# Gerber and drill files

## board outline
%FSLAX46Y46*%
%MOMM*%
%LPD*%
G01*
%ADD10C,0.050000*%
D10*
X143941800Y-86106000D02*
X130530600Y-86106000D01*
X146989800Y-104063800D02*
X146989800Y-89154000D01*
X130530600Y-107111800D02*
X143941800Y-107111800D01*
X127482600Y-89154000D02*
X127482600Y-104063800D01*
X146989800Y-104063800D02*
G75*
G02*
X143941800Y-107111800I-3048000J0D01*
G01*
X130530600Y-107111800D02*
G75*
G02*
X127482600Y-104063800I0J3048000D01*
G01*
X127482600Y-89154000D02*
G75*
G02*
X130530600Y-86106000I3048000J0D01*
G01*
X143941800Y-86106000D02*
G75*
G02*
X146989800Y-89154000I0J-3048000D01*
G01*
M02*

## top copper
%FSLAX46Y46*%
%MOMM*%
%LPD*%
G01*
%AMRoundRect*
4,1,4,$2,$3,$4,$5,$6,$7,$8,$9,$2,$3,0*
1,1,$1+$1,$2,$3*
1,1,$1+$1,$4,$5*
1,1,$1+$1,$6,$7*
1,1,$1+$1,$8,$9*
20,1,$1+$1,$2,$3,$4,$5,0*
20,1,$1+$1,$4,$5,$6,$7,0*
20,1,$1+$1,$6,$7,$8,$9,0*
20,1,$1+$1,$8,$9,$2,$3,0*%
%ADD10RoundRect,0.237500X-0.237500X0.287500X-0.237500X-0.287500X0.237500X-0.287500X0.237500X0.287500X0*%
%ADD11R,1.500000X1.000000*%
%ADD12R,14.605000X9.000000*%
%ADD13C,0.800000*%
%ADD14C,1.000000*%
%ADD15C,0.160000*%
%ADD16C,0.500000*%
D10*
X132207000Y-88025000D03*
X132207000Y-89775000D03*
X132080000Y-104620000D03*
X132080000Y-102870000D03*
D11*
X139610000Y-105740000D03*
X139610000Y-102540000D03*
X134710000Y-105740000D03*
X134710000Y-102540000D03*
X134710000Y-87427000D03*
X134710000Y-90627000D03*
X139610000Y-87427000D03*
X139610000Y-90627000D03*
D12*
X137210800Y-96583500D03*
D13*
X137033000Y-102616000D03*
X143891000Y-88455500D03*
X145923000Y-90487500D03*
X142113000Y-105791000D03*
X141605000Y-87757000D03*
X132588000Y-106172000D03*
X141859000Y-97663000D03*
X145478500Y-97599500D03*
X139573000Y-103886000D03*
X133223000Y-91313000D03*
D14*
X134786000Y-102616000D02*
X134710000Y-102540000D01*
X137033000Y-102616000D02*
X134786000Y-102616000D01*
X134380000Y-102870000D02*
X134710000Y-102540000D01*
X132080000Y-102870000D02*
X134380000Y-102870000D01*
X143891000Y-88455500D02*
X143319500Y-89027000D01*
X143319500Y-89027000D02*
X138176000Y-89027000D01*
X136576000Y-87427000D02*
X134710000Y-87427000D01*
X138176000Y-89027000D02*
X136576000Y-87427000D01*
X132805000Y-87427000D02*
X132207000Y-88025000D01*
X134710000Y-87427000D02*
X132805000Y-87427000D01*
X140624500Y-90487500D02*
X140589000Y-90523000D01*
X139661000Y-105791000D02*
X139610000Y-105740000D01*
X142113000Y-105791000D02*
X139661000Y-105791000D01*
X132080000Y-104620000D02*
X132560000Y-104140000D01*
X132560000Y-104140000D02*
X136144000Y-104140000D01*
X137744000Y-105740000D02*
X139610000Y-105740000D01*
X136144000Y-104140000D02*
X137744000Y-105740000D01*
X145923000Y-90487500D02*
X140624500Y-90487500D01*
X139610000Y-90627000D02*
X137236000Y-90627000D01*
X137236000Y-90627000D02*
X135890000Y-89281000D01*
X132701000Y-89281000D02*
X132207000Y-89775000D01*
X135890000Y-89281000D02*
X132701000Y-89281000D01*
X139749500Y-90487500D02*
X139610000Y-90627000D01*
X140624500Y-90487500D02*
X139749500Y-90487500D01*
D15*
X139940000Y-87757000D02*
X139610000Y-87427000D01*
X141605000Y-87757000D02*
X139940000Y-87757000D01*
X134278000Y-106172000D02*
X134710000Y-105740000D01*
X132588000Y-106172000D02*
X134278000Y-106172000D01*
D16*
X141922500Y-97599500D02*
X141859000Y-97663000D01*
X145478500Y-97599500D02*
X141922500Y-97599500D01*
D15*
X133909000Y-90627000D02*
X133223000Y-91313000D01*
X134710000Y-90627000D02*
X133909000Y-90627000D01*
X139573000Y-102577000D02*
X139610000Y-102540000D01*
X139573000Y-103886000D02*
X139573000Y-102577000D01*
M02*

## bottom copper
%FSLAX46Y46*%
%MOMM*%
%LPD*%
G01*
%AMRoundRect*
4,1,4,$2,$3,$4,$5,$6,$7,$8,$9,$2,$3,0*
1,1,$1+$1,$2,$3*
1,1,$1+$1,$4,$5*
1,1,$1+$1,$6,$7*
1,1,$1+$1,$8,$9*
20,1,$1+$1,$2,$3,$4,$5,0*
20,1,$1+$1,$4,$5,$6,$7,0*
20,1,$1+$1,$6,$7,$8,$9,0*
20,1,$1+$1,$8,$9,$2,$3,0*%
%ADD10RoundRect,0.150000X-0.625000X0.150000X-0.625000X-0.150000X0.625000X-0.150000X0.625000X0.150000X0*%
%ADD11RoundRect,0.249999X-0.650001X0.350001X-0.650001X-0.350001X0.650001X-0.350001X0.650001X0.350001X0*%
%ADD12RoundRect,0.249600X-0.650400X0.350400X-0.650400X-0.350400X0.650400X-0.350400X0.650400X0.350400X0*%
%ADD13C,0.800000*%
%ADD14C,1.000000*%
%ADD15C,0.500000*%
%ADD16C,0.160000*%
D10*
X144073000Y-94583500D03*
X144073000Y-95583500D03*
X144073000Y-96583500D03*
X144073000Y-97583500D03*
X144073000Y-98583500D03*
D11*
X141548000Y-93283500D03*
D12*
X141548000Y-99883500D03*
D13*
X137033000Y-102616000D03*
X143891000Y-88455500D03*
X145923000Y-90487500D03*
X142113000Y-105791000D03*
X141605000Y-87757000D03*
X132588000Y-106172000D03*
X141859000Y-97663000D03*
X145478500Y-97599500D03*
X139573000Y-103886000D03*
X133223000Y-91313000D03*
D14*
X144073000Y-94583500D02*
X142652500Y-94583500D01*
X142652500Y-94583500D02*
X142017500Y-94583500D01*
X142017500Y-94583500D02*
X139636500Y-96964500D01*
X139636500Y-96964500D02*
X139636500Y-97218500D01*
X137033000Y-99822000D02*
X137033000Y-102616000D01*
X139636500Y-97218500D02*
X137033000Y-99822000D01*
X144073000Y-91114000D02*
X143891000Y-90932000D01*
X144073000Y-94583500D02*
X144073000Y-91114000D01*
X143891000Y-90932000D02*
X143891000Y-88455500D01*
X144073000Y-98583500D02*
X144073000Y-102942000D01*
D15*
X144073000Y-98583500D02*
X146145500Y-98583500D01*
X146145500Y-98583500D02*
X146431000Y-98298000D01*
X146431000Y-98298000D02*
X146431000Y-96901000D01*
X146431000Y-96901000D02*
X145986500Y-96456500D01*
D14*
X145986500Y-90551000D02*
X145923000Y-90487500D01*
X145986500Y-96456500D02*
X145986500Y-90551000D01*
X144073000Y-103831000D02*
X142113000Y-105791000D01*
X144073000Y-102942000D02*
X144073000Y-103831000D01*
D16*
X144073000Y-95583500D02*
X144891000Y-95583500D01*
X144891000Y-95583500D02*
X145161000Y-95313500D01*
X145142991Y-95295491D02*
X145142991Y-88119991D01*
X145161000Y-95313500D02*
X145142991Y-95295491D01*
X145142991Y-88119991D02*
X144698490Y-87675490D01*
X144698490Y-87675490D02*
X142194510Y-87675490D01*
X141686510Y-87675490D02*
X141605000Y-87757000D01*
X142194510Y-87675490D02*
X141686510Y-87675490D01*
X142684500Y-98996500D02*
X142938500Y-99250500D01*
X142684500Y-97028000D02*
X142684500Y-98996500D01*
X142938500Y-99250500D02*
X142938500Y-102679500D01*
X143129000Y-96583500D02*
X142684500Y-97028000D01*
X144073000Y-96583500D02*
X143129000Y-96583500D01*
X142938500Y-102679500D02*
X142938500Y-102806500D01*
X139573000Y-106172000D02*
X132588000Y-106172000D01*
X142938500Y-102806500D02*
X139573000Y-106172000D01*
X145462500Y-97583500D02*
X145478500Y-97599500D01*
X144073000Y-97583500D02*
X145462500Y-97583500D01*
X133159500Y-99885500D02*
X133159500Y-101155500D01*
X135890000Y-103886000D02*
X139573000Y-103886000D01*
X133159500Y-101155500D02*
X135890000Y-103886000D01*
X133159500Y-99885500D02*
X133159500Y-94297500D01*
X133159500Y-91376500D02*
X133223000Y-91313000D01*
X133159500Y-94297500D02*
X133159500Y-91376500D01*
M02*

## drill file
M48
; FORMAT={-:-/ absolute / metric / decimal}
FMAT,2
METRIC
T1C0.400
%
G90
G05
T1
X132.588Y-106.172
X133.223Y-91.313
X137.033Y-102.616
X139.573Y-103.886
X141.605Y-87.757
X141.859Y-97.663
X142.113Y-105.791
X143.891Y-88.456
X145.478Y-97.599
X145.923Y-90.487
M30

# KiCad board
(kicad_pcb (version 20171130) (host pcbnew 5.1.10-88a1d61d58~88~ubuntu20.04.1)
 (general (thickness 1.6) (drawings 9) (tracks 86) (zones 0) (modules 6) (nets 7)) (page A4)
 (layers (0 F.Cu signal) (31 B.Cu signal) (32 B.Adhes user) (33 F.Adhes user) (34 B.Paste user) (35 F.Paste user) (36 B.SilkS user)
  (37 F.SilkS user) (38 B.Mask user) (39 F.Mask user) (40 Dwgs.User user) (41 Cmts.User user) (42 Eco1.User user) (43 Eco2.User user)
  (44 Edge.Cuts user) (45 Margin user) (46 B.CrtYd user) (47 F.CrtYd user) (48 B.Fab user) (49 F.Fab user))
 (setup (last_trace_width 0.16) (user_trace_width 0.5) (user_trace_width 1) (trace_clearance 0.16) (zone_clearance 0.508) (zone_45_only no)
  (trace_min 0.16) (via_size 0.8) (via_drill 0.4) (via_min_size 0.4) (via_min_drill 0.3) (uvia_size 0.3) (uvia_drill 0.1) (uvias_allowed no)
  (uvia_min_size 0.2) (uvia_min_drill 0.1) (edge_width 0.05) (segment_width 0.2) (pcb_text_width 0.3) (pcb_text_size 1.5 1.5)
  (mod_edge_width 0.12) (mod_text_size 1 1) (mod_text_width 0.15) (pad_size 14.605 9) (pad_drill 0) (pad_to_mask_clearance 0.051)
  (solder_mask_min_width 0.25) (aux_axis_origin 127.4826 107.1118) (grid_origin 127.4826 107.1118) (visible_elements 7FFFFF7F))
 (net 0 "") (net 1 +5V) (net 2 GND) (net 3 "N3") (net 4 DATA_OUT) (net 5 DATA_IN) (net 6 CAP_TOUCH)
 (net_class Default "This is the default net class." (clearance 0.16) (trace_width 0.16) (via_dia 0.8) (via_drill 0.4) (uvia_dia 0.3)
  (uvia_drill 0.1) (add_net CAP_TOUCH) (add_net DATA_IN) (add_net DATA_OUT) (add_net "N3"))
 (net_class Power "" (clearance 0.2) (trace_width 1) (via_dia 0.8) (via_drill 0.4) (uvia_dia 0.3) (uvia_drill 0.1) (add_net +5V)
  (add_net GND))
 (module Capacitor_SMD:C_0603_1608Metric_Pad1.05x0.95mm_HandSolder (layer F.Cu) (at 132.207 88.9 270)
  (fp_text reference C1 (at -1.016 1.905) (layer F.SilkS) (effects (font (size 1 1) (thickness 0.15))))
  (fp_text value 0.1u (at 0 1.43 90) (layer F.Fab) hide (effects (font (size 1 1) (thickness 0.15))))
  (pad 1 smd roundrect (at -0.875 0 270) (size 1.05 0.95) (layers F.Cu F.Paste F.Mask) (roundrect_rratio 0.25) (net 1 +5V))
  (pad 2 smd roundrect (at 0.875 0 270) (size 1.05 0.95) (layers F.Cu F.Mask) (roundrect_rratio 0.25) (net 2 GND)))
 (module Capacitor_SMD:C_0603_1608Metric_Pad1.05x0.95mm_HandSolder (layer F.Cu) (at 132.08 103.745 270)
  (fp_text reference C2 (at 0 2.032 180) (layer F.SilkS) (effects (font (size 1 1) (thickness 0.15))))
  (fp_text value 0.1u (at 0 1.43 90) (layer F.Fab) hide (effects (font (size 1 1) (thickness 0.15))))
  (pad 2 smd roundrect (at 0.875 0 270) (size 1.05 0.95) (layers F.Cu F.Mask) (roundrect_rratio 0.25) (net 2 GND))
  (pad 1 smd roundrect (at -0.875 0 270) (size 1.05 0.95) (layers F.Cu F.Paste F.Mask) (roundrect_rratio 0.25) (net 1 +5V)))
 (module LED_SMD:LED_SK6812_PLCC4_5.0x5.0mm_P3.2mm (layer F.Cu) (at 137.16 104.14)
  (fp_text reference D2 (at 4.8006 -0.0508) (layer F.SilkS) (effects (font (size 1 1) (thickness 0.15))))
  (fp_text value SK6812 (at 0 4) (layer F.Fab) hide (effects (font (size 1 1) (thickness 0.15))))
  (pad 1 smd rect (at 2.45 1.6) (size 1.5 1) (layers F.Cu F.Mask) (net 2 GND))
  (pad 2 smd rect (at 2.45 -1.6) (size 1.5 1) (layers F.Cu F.Mask) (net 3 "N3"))
  (pad 4 smd rect (at -2.45 1.6) (size 1.5 1) (layers F.Cu F.Mask) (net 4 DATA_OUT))
  (pad 3 smd rect (at -2.45 -1.6) (size 1.5 1) (layers F.Cu F.Paste F.Mask) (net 1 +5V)))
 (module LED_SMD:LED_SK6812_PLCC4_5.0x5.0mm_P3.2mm (layer F.Cu) (at 137.16 89.027)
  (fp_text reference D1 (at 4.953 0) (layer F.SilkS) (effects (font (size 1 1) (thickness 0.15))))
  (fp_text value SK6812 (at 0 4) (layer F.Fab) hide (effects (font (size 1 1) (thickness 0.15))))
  (pad 3 smd rect (at -2.45 -1.6) (size 1.5 1) (layers F.Cu F.Paste F.Mask) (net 1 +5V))
  (pad 4 smd rect (at -2.45 1.6) (size 1.5 1) (layers F.Cu F.Mask) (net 3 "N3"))
  (pad 2 smd rect (at 2.45 -1.6) (size 1.5 1) (layers F.Cu F.Mask) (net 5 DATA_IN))
  (pad 1 smd rect (at 2.45 1.6) (size 1.5 1) (layers F.Cu F.Mask) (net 2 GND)))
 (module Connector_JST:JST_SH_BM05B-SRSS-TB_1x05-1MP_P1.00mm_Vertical (layer B.Cu) (at 142.748 96.5835 270)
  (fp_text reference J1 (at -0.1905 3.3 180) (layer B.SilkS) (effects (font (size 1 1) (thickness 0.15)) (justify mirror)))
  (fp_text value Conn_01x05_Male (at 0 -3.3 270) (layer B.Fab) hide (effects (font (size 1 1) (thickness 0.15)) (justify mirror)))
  (pad 1 smd roundrect (at -2 -1.325 270) (size 0.6 1.55) (layers B.Cu B.Mask) (roundrect_rratio 0.25) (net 1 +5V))
  (pad 2 smd roundrect (at -1 -1.325 270) (size 0.6 1.55) (layers B.Cu B.Mask) (roundrect_rratio 0.25) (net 5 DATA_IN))
  (pad 3 smd roundrect (at 0 -1.325 270) (size 0.6 1.55) (layers B.Cu B.Mask) (roundrect_rratio 0.25) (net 4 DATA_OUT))
  (pad 4 smd roundrect (at 1 -1.325 270) (size 0.6 1.55) (layers B.Cu B.Mask) (roundrect_rratio 0.25) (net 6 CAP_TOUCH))
  (pad 5 smd roundrect (at 2 -1.325 270) (size 0.6 1.55) (layers B.Cu B.Mask) (roundrect_rratio 0.25) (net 2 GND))
  (pad MP smd roundrect (at -3.3 1.2 270) (size 1.2 1.8) (layers B.Cu B.Paste B.Mask) (roundrect_rratio 0.2083325))
  (pad MP smd roundrect (at 3.3 1.2 270) (size 1.2 1.8) (layers B.Cu B.Mask) (roundrect_rratio 0.208)))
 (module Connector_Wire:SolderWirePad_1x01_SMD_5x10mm (layer F.Cu) (at 136.0805 96.647)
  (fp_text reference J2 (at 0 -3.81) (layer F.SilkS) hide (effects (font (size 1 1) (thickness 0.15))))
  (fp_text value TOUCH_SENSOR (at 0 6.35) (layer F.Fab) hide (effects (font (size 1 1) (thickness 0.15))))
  (pad 1 smd rect (at 1.1303 -0.0635) (size 14.605 9) (layers F.Cu F.Mask) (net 6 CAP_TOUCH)))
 (gr_line (start 143.9418 86.106) (end 130.5306 86.106) (layer Edge.Cuts) (width 0.05))
 (gr_line (start 146.9898 104.0638) (end 146.9898 89.154) (layer Edge.Cuts) (width 0.05))
 (gr_line (start 130.5306 107.1118) (end 143.9418 107.1118) (layer Edge.Cuts) (width 0.05))
 (gr_line (start 127.4826 89.154) (end 127.4826 104.0638) (layer Edge.Cuts) (width 0.05))
 (gr_arc (start 143.9418 104.0638) (end 143.9418 107.1118) (angle -90) (layer Edge.Cuts) (width 0.05))
 (gr_arc (start 130.5306 104.0638) (end 127.4826 104.0638) (angle -90) (layer Edge.Cuts) (width 0.05))
 (gr_arc (start 130.5306 89.154) (end 130.5306 86.106) (angle -90) (layer Edge.Cuts) (width 0.05))
 (gr_arc (start 143.9418 89.154) (end 146.9898 89.154) (angle -90) (layer Edge.Cuts) (width 0.05))
 (segment (start 144.073 94.5835) (end 142.6525 94.5835) (width 1) (layer B.Cu) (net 1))
 (segment (start 142.6525 94.5835) (end 142.0175 94.5835) (width 1) (layer B.Cu) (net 1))
 (segment (start 142.0175 94.5835) (end 139.6365 96.9645) (width 1) (layer B.Cu) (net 1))
 (segment (start 139.6365 96.9645) (end 139.6365 97.2185) (width 1) (layer B.Cu) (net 1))
 (via (at 137.033 102.616) (size 0.8) (drill 0.4) (layers F.Cu B.Cu) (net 1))
 (segment (start 137.033 99.822) (end 137.033 102.616) (width 1) (layer B.Cu) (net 1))
 (segment (start 139.6365 97.2185) (end 137.033 99.822) (width 1) (layer B.Cu) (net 1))
 (segment (start 134.786 102.616) (end 134.71 102.54) (width 1) (layer F.Cu) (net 1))
 (segment (start 137.033 102.616) (end 134.786 102.616) (width 1) (layer F.Cu) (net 1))
 (segment (start 134.38 102.87) (end 134.71 102.54) (width 1) (layer F.Cu) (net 1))
 (segment (start 132.08 102.87) (end 134.38 102.87) (width 1) (layer F.Cu) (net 1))
 (via (at 143.891 88.4555) (size 0.8) (drill 0.4) (layers F.Cu B.Cu) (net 1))
 (segment (start 144.073 91.114) (end 143.891 90.932) (width 1) (layer B.Cu) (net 1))
 (segment (start 144.073 94.5835) (end 144.073 91.114) (width 1) (layer B.Cu) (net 1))
 (segment (start 143.891 90.932) (end 143.891 88.4555) (width 1) (layer B.Cu) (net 1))
 (segment (start 143.891 88.4555) (end 143.3195 89.027) (width 1) (layer F.Cu) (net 1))
 (segment (start 143.3195 89.027) (end 138.176 89.027) (width 1) (layer F.Cu) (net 1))
 (segment (start 136.576 87.427) (end 134.71 87.427) (width 1) (layer F.Cu) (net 1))
 (segment (start 138.176 89.027) (end 136.576 87.427) (width 1) (layer F.Cu) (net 1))
 (segment (start 132.805 87.427) (end 132.207 88.025) (width 1) (layer F.Cu) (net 1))
 (segment (start 134.71 87.427) (end 132.805 87.427) (width 1) (layer F.Cu) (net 1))
 (segment (start 144.073 98.5835) (end 144.073 102.942) (width 1) (layer B.Cu) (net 2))
 (segment (start 144.073 98.5835) (end 146.1455 98.5835) (width 0.5) (layer B.Cu) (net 2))
 (segment (start 146.1455 98.5835) (end 146.431 98.298) (width 0.5) (layer B.Cu) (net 2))
 (segment (start 146.431 98.298) (end 146.431 96.901) (width 0.5) (layer B.Cu) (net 2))
 (segment (start 146.431 96.901) (end 145.9865 96.4565) (width 0.5) (layer B.Cu) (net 2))
 (via (at 145.923 90.4875) (size 0.8) (drill 0.4) (layers F.Cu B.Cu) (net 2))
 (segment (start 140.6245 90.4875) (end 140.589 90.523) (width 1) (layer F.Cu) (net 2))
 (segment (start 145.9865 90.551) (end 145.923 90.4875) (width 1) (layer B.Cu) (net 2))
 (segment (start 145.9865 96.4565) (end 145.9865 90.551) (width 1) (layer B.Cu) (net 2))
 (via (at 142.113 105.791) (size 0.8) (drill 0.4) (layers F.Cu B.Cu) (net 2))
 (segment (start 144.073 103.831) (end 142.113 105.791) (width 1) (layer B.Cu) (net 2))
 (segment (start 144.073 102.942) (end 144.073 103.831) (width 1) (layer B.Cu) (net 2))
 (segment (start 139.661 105.791) (end 139.61 105.74) (width 1) (layer F.Cu) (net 2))
 (segment (start 142.113 105.791) (end 139.661 105.791) (width 1) (layer F.Cu) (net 2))
 (segment (start 132.08 104.62) (end 132.56 104.14) (width 1) (layer F.Cu) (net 2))
 (segment (start 132.56 104.14) (end 136.144 104.14) (width 1) (layer F.Cu) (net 2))
 (segment (start 137.744 105.74) (end 139.61 105.74) (width 1) (layer F.Cu) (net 2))
 (segment (start 136.144 104.14) (end 137.744 105.74) (width 1) (layer F.Cu) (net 2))
 (segment (start 145.923 90.4875) (end 140.6245 90.4875) (width 1) (layer F.Cu) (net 2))
 (segment (start 139.61 90.627) (end 137.236 90.627) (width 1) (layer F.Cu) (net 2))
 (segment (start 137.236 90.627) (end 135.89 89.281) (width 1) (layer F.Cu) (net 2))
 (segment (start 132.701 89.281) (end 132.207 89.775) (width 1) (layer F.Cu) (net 2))
 (segment (start 135.89 89.281) (end 132.701 89.281) (width 1) (layer F.Cu) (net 2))
 (segment (start 139.7495 90.4875) (end 139.61 90.627) (width 1) (layer F.Cu) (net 2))
 (segment (start 140.6245 90.4875) (end 139.7495 90.4875) (width 1) (layer F.Cu) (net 2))
 (segment (start 144.073 95.5835) (end 144.891 95.5835) (width 0.16) (layer B.Cu) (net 5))
 (segment (start 144.891 95.5835) (end 145.161 95.3135) (width 0.16) (layer B.Cu) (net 5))
 (segment (start 145.142991 95.295491) (end 145.142991 88.119991) (width 0.16) (layer B.Cu) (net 5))
 (segment (start 145.161 95.3135) (end 145.142991 95.295491) (width 0.16) (layer B.Cu) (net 5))
 (segment (start 145.142991 88.119991) (end 144.69849 87.67549) (width 0.16) (layer B.Cu) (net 5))
 (segment (start 144.69849 87.67549) (end 142.19451 87.67549) (width 0.16) (layer B.Cu) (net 5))
 (via (at 141.605 87.757) (size 0.8) (drill 0.4) (layers F.Cu B.Cu) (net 5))
 (segment (start 141.68651 87.67549) (end 141.605 87.757) (width 0.16) (layer B.Cu) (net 5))
 (segment (start 142.19451 87.67549) (end 141.68651 87.67549) (width 0.16) (layer B.Cu) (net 5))
 (segment (start 139.94 87.757) (end 139.61 87.427) (width 0.16) (layer F.Cu) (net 5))
 (segment (start 141.605 87.757) (end 139.94 87.757) (width 0.16) (layer F.Cu) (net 5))
 (segment (start 142.6845 98.9965) (end 142.9385 99.2505) (width 0.16) (layer B.Cu) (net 4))
 (segment (start 142.6845 97.028) (end 142.6845 98.9965) (width 0.16) (layer B.Cu) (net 4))
 (segment (start 142.9385 99.2505) (end 142.9385 102.6795) (width 0.16) (layer B.Cu) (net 4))
 (segment (start 143.129 96.5835) (end 142.6845 97.028) (width 0.16) (layer B.Cu) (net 4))
 (segment (start 144.073 96.5835) (end 143.129 96.5835) (width 0.16) (layer B.Cu) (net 4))
 (segment (start 142.9385 102.6795) (end 142.9385 102.8065) (width 0.16) (layer B.Cu) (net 4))
 (via (at 132.588 106.172) (size 0.8) (drill 0.4) (layers F.Cu B.Cu) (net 4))
 (segment (start 139.573 106.172) (end 132.588 106.172) (width 0.16) (layer B.Cu) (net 4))
 (segment (start 142.9385 102.8065) (end 139.573 106.172) (width 0.16) (layer B.Cu) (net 4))
 (segment (start 134.278 106.172) (end 134.71 105.74) (width 0.16) (layer F.Cu) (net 4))
 (segment (start 132.588 106.172) (end 134.278 106.172) (width 0.16) (layer F.Cu) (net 4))
 (via (at 141.859 97.663) (size 0.8) (drill 0.4) (layers F.Cu B.Cu) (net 6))
 (via (at 145.4785 97.5995) (size 0.8) (drill 0.4) (layers F.Cu B.Cu) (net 6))
 (segment (start 145.4625 97.5835) (end 145.4785 97.5995) (width 0.16) (layer B.Cu) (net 6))
 (segment (start 144.073 97.5835) (end 145.4625 97.5835) (width 0.16) (layer B.Cu) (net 6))
 (segment (start 141.9225 97.5995) (end 141.859 97.663) (width 0.5) (layer F.Cu) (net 6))
 (segment (start 145.4785 97.5995) (end 141.9225 97.5995) (width 0.5) (layer F.Cu) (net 6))
 (segment (start 133.1595 99.8855) (end 133.1595 101.1555) (width 0.16) (layer B.Cu) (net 3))
 (via (at 139.573 103.886) (size 0.8) (drill 0.4) (layers F.Cu B.Cu) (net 3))
 (segment (start 135.89 103.886) (end 139.573 103.886) (width 0.16) (layer B.Cu) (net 3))
 (segment (start 133.1595 101.1555) (end 135.89 103.886) (width 0.16) (layer B.Cu) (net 3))
 (segment (start 133.1595 99.8855) (end 133.1595 94.2975) (width 0.16) (layer B.Cu) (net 3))
 (via (at 133.223 91.313) (size 0.8) (drill 0.4) (layers F.Cu B.Cu) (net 3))
 (segment (start 133.1595 91.3765) (end 133.223 91.313) (width 0.16) (layer B.Cu) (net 3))
 (segment (start 133.1595 94.2975) (end 133.1595 91.3765) (width 0.16) (layer B.Cu) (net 3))
 (segment (start 133.909 90.627) (end 133.223 91.313) (width 0.16) (layer F.Cu) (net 3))
 (segment (start 134.71 90.627) (end 133.909 90.627) (width 0.16) (layer F.Cu) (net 3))
 (segment (start 139.573 102.577) (end 139.61 102.54) (width 0.16) (layer F.Cu) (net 3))
 (segment (start 139.573 103.886) (end 139.573 102.577) (width 0.16) (layer F.Cu) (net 3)))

